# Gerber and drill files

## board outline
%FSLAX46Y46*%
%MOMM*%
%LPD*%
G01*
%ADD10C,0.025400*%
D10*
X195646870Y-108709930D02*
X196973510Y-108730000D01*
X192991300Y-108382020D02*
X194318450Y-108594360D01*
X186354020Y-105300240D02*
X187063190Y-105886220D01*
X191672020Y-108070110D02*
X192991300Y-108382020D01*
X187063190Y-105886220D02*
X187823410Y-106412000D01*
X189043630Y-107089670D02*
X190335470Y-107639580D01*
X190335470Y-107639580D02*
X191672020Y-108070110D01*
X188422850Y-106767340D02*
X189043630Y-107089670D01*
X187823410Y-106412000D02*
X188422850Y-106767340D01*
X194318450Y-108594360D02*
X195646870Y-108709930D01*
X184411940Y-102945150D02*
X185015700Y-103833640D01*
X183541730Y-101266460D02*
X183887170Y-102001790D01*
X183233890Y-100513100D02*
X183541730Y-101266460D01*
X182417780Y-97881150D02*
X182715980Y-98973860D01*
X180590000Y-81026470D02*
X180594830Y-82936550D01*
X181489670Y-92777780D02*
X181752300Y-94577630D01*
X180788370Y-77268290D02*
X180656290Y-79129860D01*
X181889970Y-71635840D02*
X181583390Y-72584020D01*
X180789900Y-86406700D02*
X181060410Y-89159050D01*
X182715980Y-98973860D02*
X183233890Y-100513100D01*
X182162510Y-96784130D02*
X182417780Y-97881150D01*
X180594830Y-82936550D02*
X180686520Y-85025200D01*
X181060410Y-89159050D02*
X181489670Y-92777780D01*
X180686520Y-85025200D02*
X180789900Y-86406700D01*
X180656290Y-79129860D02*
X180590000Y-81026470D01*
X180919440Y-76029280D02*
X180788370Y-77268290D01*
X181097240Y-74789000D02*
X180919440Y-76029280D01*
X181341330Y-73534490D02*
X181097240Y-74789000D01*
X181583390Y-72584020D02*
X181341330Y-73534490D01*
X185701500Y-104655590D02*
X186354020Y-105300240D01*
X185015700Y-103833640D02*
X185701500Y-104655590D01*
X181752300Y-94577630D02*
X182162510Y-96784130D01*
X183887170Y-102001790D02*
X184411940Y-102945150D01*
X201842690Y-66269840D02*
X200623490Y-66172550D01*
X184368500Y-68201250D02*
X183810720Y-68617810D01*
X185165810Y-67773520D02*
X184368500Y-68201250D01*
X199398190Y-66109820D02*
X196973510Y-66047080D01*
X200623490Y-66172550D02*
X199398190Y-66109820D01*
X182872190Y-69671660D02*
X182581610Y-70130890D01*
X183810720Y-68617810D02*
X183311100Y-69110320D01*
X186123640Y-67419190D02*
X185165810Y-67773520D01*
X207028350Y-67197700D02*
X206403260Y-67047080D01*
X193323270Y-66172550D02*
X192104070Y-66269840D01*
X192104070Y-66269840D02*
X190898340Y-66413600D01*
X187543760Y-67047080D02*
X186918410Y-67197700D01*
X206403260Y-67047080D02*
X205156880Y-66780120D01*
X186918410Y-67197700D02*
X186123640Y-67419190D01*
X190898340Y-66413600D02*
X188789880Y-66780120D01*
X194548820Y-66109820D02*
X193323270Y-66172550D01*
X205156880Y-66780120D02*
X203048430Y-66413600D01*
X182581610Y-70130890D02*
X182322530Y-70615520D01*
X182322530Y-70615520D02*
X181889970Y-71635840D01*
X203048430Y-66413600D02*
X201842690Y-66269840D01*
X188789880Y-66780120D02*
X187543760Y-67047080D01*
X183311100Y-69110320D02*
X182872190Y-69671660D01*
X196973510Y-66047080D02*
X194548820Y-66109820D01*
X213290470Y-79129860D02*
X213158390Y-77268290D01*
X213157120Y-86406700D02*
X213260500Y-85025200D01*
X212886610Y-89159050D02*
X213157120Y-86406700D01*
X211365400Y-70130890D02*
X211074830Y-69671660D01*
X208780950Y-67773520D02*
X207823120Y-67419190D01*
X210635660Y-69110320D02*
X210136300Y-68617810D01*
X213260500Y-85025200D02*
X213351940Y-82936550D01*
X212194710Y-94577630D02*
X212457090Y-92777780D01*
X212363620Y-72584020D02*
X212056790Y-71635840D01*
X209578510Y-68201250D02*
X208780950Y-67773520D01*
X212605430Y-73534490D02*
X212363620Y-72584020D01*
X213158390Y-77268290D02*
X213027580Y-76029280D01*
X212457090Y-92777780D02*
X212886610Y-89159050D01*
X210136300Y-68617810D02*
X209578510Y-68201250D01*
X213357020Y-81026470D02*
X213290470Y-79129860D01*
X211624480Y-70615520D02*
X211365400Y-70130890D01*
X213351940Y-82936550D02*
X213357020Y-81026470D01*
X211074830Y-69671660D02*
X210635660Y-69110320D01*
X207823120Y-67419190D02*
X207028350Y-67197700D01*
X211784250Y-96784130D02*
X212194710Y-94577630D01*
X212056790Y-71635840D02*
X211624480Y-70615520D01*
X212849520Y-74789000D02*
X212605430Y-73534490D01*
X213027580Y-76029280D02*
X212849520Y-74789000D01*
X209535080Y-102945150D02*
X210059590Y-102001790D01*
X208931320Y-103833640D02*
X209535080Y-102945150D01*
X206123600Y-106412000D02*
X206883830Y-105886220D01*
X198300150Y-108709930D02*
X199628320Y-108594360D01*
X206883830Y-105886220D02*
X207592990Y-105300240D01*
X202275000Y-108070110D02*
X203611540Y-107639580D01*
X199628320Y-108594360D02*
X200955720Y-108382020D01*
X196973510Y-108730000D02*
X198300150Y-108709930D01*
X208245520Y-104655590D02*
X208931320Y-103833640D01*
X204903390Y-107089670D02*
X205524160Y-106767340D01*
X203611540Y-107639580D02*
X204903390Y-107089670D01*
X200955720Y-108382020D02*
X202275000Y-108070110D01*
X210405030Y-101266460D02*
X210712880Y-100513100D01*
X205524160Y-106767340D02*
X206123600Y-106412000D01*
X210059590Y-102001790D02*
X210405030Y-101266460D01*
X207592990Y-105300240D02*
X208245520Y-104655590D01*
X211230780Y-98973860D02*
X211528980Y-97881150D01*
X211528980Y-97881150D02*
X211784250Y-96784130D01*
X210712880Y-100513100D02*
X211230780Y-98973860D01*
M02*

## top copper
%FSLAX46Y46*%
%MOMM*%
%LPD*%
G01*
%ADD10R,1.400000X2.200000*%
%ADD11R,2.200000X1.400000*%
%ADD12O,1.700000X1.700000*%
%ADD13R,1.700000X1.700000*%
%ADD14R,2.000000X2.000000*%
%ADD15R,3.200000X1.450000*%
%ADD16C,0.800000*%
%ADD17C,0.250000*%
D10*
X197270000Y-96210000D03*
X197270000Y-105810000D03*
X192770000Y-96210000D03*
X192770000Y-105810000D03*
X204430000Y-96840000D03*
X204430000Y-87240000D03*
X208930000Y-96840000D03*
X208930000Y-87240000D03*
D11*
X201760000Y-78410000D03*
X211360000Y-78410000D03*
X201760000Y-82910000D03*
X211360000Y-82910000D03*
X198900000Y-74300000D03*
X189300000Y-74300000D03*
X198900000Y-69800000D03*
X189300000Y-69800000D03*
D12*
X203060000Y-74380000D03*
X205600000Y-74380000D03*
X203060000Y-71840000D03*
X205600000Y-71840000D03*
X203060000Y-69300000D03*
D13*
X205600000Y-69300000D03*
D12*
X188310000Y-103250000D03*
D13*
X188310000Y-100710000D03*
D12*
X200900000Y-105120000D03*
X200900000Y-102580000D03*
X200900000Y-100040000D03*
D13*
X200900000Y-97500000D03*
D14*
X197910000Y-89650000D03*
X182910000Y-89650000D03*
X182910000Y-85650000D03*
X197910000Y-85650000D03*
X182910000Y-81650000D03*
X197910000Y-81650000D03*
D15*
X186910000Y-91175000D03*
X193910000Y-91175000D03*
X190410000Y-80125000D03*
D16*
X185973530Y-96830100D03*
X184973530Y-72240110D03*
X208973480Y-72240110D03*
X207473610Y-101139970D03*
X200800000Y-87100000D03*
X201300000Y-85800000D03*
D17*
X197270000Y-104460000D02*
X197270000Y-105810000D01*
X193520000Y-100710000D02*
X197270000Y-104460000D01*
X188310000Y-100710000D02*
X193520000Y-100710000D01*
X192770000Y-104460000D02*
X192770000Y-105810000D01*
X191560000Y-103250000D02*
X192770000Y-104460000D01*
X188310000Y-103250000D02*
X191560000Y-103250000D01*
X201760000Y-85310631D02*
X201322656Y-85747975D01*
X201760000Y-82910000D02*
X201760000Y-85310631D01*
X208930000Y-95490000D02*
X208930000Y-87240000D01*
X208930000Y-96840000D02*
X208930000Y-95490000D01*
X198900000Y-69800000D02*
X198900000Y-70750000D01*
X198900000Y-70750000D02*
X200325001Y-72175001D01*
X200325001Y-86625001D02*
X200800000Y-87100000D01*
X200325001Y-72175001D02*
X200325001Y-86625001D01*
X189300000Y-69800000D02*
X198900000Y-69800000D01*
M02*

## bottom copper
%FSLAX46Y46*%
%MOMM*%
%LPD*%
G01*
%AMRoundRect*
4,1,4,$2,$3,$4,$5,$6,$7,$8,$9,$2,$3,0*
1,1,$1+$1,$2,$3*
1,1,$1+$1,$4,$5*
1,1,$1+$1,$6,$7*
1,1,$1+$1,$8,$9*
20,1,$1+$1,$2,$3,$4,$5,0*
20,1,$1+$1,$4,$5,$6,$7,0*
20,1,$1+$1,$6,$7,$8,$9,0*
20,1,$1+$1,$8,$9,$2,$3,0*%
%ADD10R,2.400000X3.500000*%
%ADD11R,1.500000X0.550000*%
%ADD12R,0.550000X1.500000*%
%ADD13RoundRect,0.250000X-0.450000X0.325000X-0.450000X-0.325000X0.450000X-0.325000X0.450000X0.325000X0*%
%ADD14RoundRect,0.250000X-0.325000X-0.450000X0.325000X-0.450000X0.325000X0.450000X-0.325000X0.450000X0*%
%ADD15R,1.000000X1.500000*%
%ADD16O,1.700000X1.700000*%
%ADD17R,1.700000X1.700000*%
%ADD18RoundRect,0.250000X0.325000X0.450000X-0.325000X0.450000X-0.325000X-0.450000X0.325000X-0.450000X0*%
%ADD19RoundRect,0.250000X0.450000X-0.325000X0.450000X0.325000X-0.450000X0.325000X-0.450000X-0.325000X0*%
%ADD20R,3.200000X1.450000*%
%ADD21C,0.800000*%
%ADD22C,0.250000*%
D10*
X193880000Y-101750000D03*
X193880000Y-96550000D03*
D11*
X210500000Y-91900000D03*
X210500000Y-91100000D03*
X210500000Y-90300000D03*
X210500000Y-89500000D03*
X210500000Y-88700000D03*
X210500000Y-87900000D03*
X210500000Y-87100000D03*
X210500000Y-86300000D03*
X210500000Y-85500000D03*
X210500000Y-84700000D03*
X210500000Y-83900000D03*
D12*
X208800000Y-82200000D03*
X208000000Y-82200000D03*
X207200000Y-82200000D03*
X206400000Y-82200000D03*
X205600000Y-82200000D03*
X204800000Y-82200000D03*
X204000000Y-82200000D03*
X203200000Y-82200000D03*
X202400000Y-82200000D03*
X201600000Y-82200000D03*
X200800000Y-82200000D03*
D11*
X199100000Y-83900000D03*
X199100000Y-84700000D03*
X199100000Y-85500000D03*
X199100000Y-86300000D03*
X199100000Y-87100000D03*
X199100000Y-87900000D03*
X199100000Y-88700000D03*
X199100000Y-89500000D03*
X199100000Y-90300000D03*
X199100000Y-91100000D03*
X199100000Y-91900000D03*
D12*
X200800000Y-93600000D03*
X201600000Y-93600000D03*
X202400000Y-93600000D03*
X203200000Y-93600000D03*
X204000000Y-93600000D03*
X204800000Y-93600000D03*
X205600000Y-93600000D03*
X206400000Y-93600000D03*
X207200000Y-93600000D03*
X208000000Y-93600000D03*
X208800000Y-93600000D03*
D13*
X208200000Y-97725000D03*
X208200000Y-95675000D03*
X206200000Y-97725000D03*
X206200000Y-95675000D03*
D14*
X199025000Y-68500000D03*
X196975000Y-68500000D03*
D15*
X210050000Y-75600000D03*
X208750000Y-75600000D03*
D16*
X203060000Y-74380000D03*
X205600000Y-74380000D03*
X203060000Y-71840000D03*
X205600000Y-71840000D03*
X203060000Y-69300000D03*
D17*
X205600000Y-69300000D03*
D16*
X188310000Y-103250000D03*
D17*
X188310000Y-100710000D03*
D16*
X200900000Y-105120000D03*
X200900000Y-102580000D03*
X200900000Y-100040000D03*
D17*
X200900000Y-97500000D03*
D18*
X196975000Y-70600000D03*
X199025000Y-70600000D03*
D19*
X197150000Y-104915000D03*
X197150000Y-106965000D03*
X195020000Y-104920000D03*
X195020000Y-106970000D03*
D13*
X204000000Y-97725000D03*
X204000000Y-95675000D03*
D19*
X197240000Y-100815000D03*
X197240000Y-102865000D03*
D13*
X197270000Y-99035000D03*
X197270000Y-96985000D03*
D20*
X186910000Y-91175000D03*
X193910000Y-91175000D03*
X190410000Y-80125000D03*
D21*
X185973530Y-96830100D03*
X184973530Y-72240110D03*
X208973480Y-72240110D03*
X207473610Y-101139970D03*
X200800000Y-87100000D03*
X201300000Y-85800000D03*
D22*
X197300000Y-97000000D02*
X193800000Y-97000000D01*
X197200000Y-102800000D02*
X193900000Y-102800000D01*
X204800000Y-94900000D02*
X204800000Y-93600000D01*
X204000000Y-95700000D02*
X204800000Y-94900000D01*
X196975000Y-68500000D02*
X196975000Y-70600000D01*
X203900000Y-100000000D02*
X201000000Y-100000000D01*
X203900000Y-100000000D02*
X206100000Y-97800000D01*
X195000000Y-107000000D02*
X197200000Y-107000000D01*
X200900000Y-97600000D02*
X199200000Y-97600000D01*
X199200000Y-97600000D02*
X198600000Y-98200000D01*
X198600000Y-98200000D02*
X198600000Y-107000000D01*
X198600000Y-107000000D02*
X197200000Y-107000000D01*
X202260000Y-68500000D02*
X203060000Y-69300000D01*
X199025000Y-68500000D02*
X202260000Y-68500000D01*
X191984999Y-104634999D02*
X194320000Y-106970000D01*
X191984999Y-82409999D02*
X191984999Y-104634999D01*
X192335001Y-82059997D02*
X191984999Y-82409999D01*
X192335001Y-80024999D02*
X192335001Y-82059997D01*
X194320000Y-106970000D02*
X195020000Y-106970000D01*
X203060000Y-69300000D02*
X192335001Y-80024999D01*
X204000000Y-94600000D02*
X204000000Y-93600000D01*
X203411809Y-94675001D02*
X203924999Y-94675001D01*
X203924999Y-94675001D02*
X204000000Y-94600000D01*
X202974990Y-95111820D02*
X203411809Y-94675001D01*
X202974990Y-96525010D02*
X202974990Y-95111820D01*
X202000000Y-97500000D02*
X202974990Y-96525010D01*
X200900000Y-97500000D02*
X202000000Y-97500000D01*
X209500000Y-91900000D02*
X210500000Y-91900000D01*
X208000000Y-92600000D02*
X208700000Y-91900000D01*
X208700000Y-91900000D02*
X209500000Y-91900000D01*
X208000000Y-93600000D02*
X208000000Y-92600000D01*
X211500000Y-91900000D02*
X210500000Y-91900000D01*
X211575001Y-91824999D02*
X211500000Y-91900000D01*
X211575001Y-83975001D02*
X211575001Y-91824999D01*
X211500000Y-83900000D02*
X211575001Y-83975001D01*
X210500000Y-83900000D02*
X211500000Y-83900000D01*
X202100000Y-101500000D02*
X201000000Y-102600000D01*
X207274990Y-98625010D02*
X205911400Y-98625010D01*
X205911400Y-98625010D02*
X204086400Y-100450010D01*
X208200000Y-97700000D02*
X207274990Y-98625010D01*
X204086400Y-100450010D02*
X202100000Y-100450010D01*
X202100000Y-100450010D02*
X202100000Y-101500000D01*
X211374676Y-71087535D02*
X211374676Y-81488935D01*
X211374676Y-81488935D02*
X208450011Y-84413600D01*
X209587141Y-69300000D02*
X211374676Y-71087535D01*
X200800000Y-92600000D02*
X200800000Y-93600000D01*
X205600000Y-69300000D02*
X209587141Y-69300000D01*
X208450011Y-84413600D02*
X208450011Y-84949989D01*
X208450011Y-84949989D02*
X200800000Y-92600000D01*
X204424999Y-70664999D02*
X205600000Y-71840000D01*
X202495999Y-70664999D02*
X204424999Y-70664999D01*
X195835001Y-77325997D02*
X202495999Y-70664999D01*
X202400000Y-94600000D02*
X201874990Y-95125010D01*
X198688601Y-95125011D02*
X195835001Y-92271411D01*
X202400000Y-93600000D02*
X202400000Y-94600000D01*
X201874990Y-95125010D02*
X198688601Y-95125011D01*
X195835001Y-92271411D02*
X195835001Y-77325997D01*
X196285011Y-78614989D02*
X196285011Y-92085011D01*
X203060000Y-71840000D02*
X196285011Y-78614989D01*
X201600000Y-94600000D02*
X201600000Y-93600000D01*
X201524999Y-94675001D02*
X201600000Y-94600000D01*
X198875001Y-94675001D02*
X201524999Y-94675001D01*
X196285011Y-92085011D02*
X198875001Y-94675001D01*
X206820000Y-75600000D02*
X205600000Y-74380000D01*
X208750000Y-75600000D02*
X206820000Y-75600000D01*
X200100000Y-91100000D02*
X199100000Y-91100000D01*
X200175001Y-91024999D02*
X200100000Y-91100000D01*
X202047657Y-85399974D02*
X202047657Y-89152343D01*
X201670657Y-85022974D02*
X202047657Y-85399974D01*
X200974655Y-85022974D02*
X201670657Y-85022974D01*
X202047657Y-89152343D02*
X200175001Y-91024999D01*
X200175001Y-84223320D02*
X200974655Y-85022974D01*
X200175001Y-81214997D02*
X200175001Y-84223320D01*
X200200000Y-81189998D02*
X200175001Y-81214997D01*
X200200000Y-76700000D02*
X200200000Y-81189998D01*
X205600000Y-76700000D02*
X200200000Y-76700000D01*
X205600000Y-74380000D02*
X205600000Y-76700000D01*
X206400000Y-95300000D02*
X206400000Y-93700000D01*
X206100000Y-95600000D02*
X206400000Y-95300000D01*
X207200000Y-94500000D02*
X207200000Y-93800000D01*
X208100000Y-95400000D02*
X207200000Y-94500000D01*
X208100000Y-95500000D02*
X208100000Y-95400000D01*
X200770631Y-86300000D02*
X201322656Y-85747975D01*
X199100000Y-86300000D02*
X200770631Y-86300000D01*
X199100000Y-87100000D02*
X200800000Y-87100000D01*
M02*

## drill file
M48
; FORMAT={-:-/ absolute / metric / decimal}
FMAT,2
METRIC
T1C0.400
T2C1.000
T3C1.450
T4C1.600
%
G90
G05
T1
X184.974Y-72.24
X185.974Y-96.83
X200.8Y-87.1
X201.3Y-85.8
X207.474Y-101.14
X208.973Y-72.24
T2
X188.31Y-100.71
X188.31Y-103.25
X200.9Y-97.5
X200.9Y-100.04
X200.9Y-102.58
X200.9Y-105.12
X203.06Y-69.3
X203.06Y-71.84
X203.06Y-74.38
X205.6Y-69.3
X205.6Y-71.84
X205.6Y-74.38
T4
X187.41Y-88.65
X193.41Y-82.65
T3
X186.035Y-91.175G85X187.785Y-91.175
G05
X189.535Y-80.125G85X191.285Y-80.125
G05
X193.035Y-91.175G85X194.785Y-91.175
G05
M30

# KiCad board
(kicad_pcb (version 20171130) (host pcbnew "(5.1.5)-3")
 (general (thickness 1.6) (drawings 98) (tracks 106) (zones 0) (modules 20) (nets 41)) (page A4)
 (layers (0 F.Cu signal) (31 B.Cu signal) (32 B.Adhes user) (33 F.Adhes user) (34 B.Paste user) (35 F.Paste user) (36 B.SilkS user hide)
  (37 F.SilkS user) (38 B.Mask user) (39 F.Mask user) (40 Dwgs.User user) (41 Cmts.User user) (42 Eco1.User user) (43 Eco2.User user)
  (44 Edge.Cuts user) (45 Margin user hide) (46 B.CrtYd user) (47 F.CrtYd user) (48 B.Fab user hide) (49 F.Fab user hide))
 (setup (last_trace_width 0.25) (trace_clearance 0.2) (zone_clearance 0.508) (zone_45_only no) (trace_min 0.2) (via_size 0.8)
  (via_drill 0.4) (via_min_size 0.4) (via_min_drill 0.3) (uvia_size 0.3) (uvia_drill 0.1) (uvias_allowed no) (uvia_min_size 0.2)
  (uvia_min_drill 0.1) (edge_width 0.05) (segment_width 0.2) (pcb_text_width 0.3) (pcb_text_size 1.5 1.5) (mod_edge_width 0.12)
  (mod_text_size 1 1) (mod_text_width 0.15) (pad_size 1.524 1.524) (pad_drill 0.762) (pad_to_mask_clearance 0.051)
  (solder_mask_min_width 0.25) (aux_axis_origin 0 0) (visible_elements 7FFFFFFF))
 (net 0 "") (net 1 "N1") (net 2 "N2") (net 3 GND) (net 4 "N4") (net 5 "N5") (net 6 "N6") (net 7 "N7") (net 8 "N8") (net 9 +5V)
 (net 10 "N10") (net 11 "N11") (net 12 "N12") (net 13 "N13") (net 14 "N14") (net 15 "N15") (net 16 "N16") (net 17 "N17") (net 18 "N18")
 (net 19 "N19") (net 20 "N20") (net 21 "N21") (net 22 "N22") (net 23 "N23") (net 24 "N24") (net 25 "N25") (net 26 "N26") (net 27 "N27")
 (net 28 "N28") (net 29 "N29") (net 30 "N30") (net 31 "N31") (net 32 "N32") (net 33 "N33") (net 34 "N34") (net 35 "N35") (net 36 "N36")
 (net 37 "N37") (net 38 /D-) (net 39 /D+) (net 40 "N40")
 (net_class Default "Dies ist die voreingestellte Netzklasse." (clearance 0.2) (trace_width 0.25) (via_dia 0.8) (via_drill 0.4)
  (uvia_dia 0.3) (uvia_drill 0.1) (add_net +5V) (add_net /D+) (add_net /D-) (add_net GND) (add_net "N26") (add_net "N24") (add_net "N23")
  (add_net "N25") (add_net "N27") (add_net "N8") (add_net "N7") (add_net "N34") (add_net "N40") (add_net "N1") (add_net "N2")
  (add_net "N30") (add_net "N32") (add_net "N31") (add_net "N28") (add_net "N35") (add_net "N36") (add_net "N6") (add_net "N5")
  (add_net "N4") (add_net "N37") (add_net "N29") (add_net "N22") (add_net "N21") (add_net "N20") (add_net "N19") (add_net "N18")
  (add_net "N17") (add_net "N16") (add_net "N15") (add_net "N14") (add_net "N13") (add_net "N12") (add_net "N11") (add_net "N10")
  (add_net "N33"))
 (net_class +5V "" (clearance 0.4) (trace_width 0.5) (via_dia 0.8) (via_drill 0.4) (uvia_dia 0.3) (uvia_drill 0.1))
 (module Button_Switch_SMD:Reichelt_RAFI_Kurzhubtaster (layer F.Cu) (at 197.97 106.91 90)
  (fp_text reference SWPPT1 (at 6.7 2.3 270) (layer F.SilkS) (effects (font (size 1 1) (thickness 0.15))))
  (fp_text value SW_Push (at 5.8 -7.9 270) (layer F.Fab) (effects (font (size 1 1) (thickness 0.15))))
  (pad 2 smd rect (at 10.7 -0.7 90) (size 2.2 1.4) (layers F.Cu F.Paste F.Mask) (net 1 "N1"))
  (pad 2 smd rect (at 1.1 -0.7 90) (size 2.2 1.4) (layers F.Cu F.Paste F.Mask) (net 1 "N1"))
  (pad 1 smd rect (at 10.7 -5.2 90) (size 2.2 1.4) (layers F.Cu F.Paste F.Mask) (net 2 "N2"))
  (pad 1 smd rect (at 1.1 -5.2 90) (size 2.2 1.4) (layers F.Cu F.Paste F.Mask) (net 2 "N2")))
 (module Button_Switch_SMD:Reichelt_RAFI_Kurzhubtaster (layer F.Cu) (at 203.73 86.14 270)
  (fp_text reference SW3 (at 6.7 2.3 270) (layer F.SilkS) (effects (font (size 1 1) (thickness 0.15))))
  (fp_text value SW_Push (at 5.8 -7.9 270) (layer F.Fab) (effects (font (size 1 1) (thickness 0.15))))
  (pad 2 smd rect (at 10.7 -0.7 270) (size 2.2 1.4) (layers F.Cu F.Paste F.Mask) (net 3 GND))
  (pad 2 smd rect (at 1.1 -0.7 270) (size 2.2 1.4) (layers F.Cu F.Paste F.Mask) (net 3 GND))
  (pad 1 smd rect (at 10.7 -5.2 270) (size 2.2 1.4) (layers F.Cu F.Paste F.Mask) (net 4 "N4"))
  (pad 1 smd rect (at 1.1 -5.2 270) (size 2.2 1.4) (layers F.Cu F.Paste F.Mask) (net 4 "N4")))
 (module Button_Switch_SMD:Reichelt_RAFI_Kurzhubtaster (layer F.Cu) (at 212.46 77.71 180)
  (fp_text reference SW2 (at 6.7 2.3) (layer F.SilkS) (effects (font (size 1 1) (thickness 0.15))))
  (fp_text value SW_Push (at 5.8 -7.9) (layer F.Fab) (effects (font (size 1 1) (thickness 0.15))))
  (pad 2 smd rect (at 10.7 -0.7 180) (size 2.2 1.4) (layers F.Cu F.Paste F.Mask) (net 3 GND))
  (pad 2 smd rect (at 1.1 -0.7 180) (size 2.2 1.4) (layers F.Cu F.Paste F.Mask) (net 3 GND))
  (pad 1 smd rect (at 10.7 -5.2 180) (size 2.2 1.4) (layers F.Cu F.Paste F.Mask) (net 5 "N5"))
  (pad 1 smd rect (at 1.1 -5.2 180) (size 2.2 1.4) (layers F.Cu F.Paste F.Mask) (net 5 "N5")))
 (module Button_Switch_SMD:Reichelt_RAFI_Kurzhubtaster (layer F.Cu) (at 188.2 75)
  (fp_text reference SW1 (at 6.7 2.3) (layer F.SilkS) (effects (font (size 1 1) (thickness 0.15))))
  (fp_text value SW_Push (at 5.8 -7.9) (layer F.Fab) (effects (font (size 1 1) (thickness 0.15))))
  (pad 2 smd rect (at 10.7 -0.7) (size 2.2 1.4) (layers F.Cu F.Paste F.Mask) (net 3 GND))
  (pad 2 smd rect (at 1.1 -0.7) (size 2.2 1.4) (layers F.Cu F.Paste F.Mask) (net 3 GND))
  (pad 1 smd rect (at 10.7 -5.2) (size 2.2 1.4) (layers F.Cu F.Paste F.Mask) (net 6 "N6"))
  (pad 1 smd rect (at 1.1 -5.2) (size 2.2 1.4) (layers F.Cu F.Paste F.Mask) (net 6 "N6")))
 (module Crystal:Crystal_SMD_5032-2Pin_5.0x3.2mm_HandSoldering (layer B.Cu) (at 193.88 99.15 270)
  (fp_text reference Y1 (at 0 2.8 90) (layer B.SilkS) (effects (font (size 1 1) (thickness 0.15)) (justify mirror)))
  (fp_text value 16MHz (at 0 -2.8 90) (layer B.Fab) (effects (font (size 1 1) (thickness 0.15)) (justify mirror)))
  (pad 2 smd rect (at 2.6 0 270) (size 3.5 2.4) (layers B.Cu B.Paste B.Mask) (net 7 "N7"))
  (pad 1 smd rect (at -2.6 0 270) (size 3.5 2.4) (layers B.Cu B.Paste B.Mask) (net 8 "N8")))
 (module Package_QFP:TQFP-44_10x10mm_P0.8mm (layer B.Cu) (at 204.8 87.9 90)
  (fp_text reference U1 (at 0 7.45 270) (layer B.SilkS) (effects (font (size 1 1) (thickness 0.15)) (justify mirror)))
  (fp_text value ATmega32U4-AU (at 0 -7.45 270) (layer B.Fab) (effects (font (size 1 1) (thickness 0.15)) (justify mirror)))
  (pad 44 smd rect (at -4 5.7) (size 1.5 0.55) (layers B.Cu B.Paste B.Mask) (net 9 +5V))
  (pad 43 smd rect (at -3.2 5.7) (size 1.5 0.55) (layers B.Cu B.Paste B.Mask) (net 3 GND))
  (pad 42 smd rect (at -2.4 5.7) (size 1.5 0.55) (layers B.Cu B.Paste B.Mask) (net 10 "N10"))
  (pad 41 smd rect (at -1.6 5.7) (size 1.5 0.55) (layers B.Cu B.Paste B.Mask) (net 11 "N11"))
  (pad 40 smd rect (at -0.8 5.7) (size 1.5 0.55) (layers B.Cu B.Paste B.Mask) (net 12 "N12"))
  (pad 39 smd rect (at 0 5.7) (size 1.5 0.55) (layers B.Cu B.Paste B.Mask) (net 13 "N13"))
  (pad 38 smd rect (at 0.8 5.7) (size 1.5 0.55) (layers B.Cu B.Paste B.Mask) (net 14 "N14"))
  (pad 37 smd rect (at 1.6 5.7) (size 1.5 0.55) (layers B.Cu B.Paste B.Mask) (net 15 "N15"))
  (pad 36 smd rect (at 2.4 5.7) (size 1.5 0.55) (layers B.Cu B.Paste B.Mask) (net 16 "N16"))
  (pad 35 smd rect (at 3.2 5.7) (size 1.5 0.55) (layers B.Cu B.Paste B.Mask) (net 3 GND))
  (pad 34 smd rect (at 4 5.7) (size 1.5 0.55) (layers B.Cu B.Paste B.Mask) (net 9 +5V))
  (pad 33 smd rect (at 5.7 4 90) (size 1.5 0.55) (layers B.Cu B.Paste B.Mask) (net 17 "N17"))
  (pad 32 smd rect (at 5.7 3.2 90) (size 1.5 0.55) (layers B.Cu B.Paste B.Mask) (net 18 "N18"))
  (pad 31 smd rect (at 5.7 2.4 90) (size 1.5 0.55) (layers B.Cu B.Paste B.Mask) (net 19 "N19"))
  (pad 30 smd rect (at 5.7 1.6 90) (size 1.5 0.55) (layers B.Cu B.Paste B.Mask) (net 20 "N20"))
  (pad 29 smd rect (at 5.7 0.8 90) (size 1.5 0.55) (layers B.Cu B.Paste B.Mask) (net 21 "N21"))
  (pad 28 smd rect (at 5.7 0 90) (size 1.5 0.55) (layers B.Cu B.Paste B.Mask) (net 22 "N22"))
  (pad 27 smd rect (at 5.7 -0.8 90) (size 1.5 0.55) (layers B.Cu B.Paste B.Mask) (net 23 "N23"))
  (pad 26 smd rect (at 5.7 -1.6 90) (size 1.5 0.55) (layers B.Cu B.Paste B.Mask) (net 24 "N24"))
  (pad 25 smd rect (at 5.7 -2.4 90) (size 1.5 0.55) (layers B.Cu B.Paste B.Mask) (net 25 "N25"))
  (pad 24 smd rect (at 5.7 -3.2 90) (size 1.5 0.55) (layers B.Cu B.Paste B.Mask) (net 9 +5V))
  (pad 23 smd rect (at 5.7 -4 90) (size 1.5 0.55) (layers B.Cu B.Paste B.Mask) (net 3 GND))
  (pad 22 smd rect (at 4 -5.7) (size 1.5 0.55) (layers B.Cu B.Paste B.Mask) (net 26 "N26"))
  (pad 21 smd rect (at 3.2 -5.7) (size 1.5 0.55) (layers B.Cu B.Paste B.Mask) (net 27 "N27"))
  (pad 20 smd rect (at 2.4 -5.7) (size 1.5 0.55) (layers B.Cu B.Paste B.Mask) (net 4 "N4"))
  (pad 19 smd rect (at 1.6 -5.7) (size 1.5 0.55) (layers B.Cu B.Paste B.Mask) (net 5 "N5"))
  (pad 18 smd rect (at 0.8 -5.7) (size 1.5 0.55) (layers B.Cu B.Paste B.Mask) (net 6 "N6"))
  (pad 17 smd rect (at 0 -5.7) (size 1.5 0.55) (layers B.Cu B.Paste B.Mask) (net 8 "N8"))
  (pad 16 smd rect (at -0.8 -5.7) (size 1.5 0.55) (layers B.Cu B.Paste B.Mask) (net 7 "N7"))
  (pad 15 smd rect (at -1.6 -5.7) (size 1.5 0.55) (layers B.Cu B.Paste B.Mask) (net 3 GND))
  (pad 14 smd rect (at -2.4 -5.7) (size 1.5 0.55) (layers B.Cu B.Paste B.Mask) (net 9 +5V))
  (pad 13 smd rect (at -3.2 -5.7) (size 1.5 0.55) (layers B.Cu B.Paste B.Mask) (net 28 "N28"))
  (pad 12 smd rect (at -4 -5.7) (size 1.5 0.55) (layers B.Cu B.Paste B.Mask) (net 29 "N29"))
  (pad 11 smd rect (at -5.7 -4 90) (size 1.5 0.55) (layers B.Cu B.Paste B.Mask) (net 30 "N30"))
  (pad 10 smd rect (at -5.7 -3.2 90) (size 1.5 0.55) (layers B.Cu B.Paste B.Mask) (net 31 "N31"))
  (pad 9 smd rect (at -5.7 -2.4 90) (size 1.5 0.55) (layers B.Cu B.Paste B.Mask) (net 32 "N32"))
  (pad 8 smd rect (at -5.7 -1.6 90) (size 1.5 0.55) (layers B.Cu B.Paste B.Mask) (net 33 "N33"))
  (pad 7 smd rect (at -5.7 -0.8 90) (size 1.5 0.55) (layers B.Cu B.Paste B.Mask) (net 9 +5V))
  (pad 6 smd rect (at -5.7 0 90) (size 1.5 0.55) (layers B.Cu B.Paste B.Mask) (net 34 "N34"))
  (pad 5 smd rect (at -5.7 0.8 90) (size 1.5 0.55) (layers B.Cu B.Paste B.Mask) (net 3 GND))
  (pad 4 smd rect (at -5.7 1.6 90) (size 1.5 0.55) (layers B.Cu B.Paste B.Mask) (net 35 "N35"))
  (pad 3 smd rect (at -5.7 2.4 90) (size 1.5 0.55) (layers B.Cu B.Paste B.Mask) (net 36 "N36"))
  (pad 2 smd rect (at -5.7 3.2 90) (size 1.5 0.55) (layers B.Cu B.Paste B.Mask) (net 9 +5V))
  (pad 1 smd rect (at -5.7 4 90) (size 1.5 0.55) (layers B.Cu B.Paste B.Mask) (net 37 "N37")))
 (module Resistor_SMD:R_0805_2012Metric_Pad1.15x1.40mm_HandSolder (layer B.Cu) (at 208.2 96.7 270)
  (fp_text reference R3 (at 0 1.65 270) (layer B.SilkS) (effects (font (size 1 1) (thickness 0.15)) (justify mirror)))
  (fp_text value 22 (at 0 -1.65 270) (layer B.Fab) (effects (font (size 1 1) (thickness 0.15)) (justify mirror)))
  (pad 2 smd roundrect (at 1.025 0 270) (size 1.15 1.4) (layers B.Cu B.Paste B.Mask) (roundrect_rratio 0.217391) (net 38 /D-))
  (pad 1 smd roundrect (at -1.025 0 270) (size 1.15 1.4) (layers B.Cu B.Paste B.Mask) (roundrect_rratio 0.217391) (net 36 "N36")))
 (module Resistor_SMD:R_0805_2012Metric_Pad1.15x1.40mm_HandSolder (layer B.Cu) (at 206.2 96.7 270)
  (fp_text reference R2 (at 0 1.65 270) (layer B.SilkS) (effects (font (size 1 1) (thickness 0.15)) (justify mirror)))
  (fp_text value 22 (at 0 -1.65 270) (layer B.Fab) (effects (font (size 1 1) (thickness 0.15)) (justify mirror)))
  (pad 2 smd roundrect (at 1.025 0 270) (size 1.15 1.4) (layers B.Cu B.Paste B.Mask) (roundrect_rratio 0.217391) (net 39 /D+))
  (pad 1 smd roundrect (at -1.025 0 270) (size 1.15 1.4) (layers B.Cu B.Paste B.Mask) (roundrect_rratio 0.217391) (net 35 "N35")))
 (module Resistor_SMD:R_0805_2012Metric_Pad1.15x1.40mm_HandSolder (layer B.Cu) (at 198 68.5)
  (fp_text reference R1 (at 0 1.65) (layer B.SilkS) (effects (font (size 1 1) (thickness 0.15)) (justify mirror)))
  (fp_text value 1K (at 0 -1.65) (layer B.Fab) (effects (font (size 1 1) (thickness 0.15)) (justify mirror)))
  (pad 2 smd roundrect (at 1.025 0) (size 1.15 1.4) (layers B.Cu B.Paste B.Mask) (roundrect_rratio 0.217391) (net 9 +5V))
  (pad 1 smd roundrect (at -1.025 0) (size 1.15 1.4) (layers B.Cu B.Paste B.Mask) (roundrect_rratio 0.217391) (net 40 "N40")))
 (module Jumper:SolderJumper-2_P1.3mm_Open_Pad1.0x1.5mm (layer B.Cu) (at 209.4 75.6 180)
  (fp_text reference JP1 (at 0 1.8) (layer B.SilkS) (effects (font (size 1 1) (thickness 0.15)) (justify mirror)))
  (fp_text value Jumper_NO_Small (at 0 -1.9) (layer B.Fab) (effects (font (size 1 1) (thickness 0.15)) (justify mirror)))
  (pad 1 smd rect (at -0.65 0 180) (size 1 1.5) (layers B.Cu B.Mask) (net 3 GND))
  (pad 2 smd rect (at 0.65 0 180) (size 1 1.5) (layers B.Cu B.Mask) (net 28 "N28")))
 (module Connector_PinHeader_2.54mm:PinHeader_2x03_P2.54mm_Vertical (layer B.Cu) (at 205.6 69.3 180)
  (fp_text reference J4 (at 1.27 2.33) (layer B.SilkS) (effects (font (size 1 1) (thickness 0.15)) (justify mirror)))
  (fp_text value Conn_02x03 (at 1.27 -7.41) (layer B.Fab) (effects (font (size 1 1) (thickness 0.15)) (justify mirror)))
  (pad 6 thru_hole oval (at 2.54 -5.08 180) (size 1.7 1.7) (drill 1) (layers *.Cu *.Mask) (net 3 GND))
  (pad 5 thru_hole oval (at 0 -5.08 180) (size 1.7 1.7) (drill 1) (layers *.Cu *.Mask) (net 28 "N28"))
  (pad 4 thru_hole oval (at 2.54 -2.54 180) (size 1.7 1.7) (drill 1) (layers *.Cu *.Mask) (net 31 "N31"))
  (pad 3 thru_hole oval (at 0 -2.54 180) (size 1.7 1.7) (drill 1) (layers *.Cu *.Mask) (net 32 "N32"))
  (pad 2 thru_hole oval (at 2.54 0 180) (size 1.7 1.7) (drill 1) (layers *.Cu *.Mask) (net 9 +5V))
  (pad 1 thru_hole rect (at 0 0 180) (size 1.7 1.7) (drill 1) (layers *.Cu *.Mask) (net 30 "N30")))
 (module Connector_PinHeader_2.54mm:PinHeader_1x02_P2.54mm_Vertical (layer B.Cu) (at 188.31 100.71 180)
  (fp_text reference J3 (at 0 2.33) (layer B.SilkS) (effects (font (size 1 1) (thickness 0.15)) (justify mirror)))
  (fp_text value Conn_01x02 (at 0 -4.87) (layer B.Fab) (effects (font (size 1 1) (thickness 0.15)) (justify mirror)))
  (pad 2 thru_hole oval (at 0 -2.54 180) (size 1.7 1.7) (drill 1) (layers *.Cu *.Mask) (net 2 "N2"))
  (pad 1 thru_hole rect (at 0 0 180) (size 1.7 1.7) (drill 1) (layers *.Cu *.Mask) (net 1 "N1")))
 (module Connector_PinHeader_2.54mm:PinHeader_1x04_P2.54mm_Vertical (layer B.Cu) (at 200.9 97.5 180)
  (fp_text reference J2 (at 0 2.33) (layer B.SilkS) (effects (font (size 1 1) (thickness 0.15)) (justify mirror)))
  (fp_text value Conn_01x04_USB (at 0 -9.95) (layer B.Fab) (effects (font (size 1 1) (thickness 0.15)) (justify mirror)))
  (pad 4 thru_hole oval (at 0 -7.62 180) (size 1.7 1.7) (drill 1) (layers *.Cu *.Mask) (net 3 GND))
  (pad 3 thru_hole oval (at 0 -5.08 180) (size 1.7 1.7) (drill 1) (layers *.Cu *.Mask) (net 38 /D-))
  (pad 2 thru_hole oval (at 0 -2.54 180) (size 1.7 1.7) (drill 1) (layers *.Cu *.Mask) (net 39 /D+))
  (pad 1 thru_hole rect (at 0 0 180) (size 1.7 1.7) (drill 1) (layers *.Cu *.Mask) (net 9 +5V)))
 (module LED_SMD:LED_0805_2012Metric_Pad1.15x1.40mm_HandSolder (layer B.Cu) (at 198 70.6 180)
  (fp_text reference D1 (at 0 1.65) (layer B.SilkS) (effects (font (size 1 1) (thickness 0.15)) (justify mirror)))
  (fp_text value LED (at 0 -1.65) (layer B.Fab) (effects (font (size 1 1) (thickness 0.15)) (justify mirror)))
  (pad 2 smd roundrect (at 1.025 0 180) (size 1.15 1.4) (layers B.Cu B.Paste B.Mask) (roundrect_rratio 0.217391) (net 40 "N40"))
  (pad 1 smd roundrect (at -1.025 0 180) (size 1.15 1.4) (layers B.Cu B.Paste B.Mask) (roundrect_rratio 0.217391) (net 3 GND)))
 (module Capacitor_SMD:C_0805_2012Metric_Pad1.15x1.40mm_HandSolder (layer B.Cu) (at 197.15 105.94 90)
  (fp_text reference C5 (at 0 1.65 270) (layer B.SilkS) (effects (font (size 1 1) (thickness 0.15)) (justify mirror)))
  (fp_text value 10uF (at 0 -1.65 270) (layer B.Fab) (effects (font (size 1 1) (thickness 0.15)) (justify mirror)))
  (pad 2 smd roundrect (at 1.025 0 90) (size 1.15 1.4) (layers B.Cu B.Paste B.Mask) (roundrect_rratio 0.217391) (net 3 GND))
  (pad 1 smd roundrect (at -1.025 0 90) (size 1.15 1.4) (layers B.Cu B.Paste B.Mask) (roundrect_rratio 0.217391) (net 9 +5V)))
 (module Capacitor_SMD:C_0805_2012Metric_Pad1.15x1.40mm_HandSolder (layer B.Cu) (at 195.02 105.945 90)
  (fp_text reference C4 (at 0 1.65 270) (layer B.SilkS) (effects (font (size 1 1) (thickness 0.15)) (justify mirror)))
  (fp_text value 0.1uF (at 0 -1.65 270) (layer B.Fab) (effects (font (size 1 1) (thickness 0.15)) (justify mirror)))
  (pad 2 smd roundrect (at 1.025 0 90) (size 1.15 1.4) (layers B.Cu B.Paste B.Mask) (roundrect_rratio 0.217391) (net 3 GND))
  (pad 1 smd roundrect (at -1.025 0 90) (size 1.15 1.4) (layers B.Cu B.Paste B.Mask) (roundrect_rratio 0.217391) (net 9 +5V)))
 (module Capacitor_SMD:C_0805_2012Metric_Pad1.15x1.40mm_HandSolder (layer B.Cu) (at 204 96.7 270)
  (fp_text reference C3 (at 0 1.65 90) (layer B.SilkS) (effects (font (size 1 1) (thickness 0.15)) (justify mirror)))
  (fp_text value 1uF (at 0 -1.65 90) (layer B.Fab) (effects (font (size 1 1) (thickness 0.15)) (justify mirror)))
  (pad 2 smd roundrect (at 1.025 0 270) (size 1.15 1.4) (layers B.Cu B.Paste B.Mask) (roundrect_rratio 0.217391) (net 3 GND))
  (pad 1 smd roundrect (at -1.025 0 270) (size 1.15 1.4) (layers B.Cu B.Paste B.Mask) (roundrect_rratio 0.217391) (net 34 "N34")))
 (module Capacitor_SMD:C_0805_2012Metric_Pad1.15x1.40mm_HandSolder (layer B.Cu) (at 197.24 101.84 90)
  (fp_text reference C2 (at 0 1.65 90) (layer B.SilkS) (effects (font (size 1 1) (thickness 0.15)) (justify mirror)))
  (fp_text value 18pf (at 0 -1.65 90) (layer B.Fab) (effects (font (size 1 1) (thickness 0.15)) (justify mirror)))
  (pad 2 smd roundrect (at 1.025 0 90) (size 1.15 1.4) (layers B.Cu B.Paste B.Mask) (roundrect_rratio 0.217391) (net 3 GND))
  (pad 1 smd roundrect (at -1.025 0 90) (size 1.15 1.4) (layers B.Cu B.Paste B.Mask) (roundrect_rratio 0.217391) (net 7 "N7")))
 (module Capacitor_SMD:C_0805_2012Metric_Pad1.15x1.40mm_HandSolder (layer B.Cu) (at 197.27 98.01 270)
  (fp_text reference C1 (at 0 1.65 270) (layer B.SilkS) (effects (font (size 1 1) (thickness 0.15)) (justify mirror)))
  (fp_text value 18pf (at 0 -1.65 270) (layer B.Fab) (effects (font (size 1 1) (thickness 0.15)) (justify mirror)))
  (pad 2 smd roundrect (at 1.025 0 270) (size 1.15 1.4) (layers B.Cu B.Paste B.Mask) (roundrect_rratio 0.217391) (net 3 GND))
  (pad 1 smd roundrect (at -1.025 0 270) (size 1.15 1.4) (layers B.Cu B.Paste B.Mask) (roundrect_rratio 0.217391) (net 8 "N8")))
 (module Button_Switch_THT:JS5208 (layer F.Cu) (at 190.41 85.65)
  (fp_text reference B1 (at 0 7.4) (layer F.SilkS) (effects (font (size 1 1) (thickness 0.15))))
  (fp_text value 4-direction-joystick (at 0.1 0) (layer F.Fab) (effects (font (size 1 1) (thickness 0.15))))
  (pad 6 smd rect (at 7.5 4) (size 2 2) (layers F.Cu F.Paste F.Mask) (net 3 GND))
  (pad 3 smd rect (at -7.5 4) (size 2 2) (layers F.Cu F.Paste F.Mask) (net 23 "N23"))
  (pad 2 smd rect (at -7.5 0) (size 2 2) (layers F.Cu F.Paste F.Mask) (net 24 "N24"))
  (pad 5 smd rect (at 7.5 0) (size 2 2) (layers F.Cu F.Paste F.Mask) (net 27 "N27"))
  (pad 1 smd rect (at -7.5 -4) (size 2 2) (layers F.Cu F.Paste F.Mask) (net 26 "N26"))
  (pad 4 smd rect (at 7.5 -4) (size 2 2) (layers F.Cu F.Paste F.Mask) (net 25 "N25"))
  (pad "" np_thru_hole rect (at -3.5 5.525) (size 3.2 1.45) (drill oval 3.2 1.45) (layers *.Cu *.Mask))
  (pad "" np_thru_hole rect (at 3.5 5.525) (size 3.2 1.45) (drill oval 3.2 1.45) (layers *.Cu *.Mask))
  (pad "" np_thru_hole rect (at 0 -5.525) (size 3.2 1.45) (drill oval 3.2 1.45) (layers *.Cu *.Mask))
  (pad "" np_thru_hole circle (at -3 3) (size 1.6 1.6) (drill 1.6) (layers *.Cu *.Mask))
  (pad "" np_thru_hole circle (at 3 -3) (size 1.6 1.6) (drill 1.6) (layers *.Cu *.Mask)))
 (gr_line (start 195.64687 108.70993) (end 196.97351 108.73) (layer Edge.Cuts) (width 0.0254))
 (gr_line (start 192.9913 108.38202) (end 194.31845 108.59436) (layer Edge.Cuts) (width 0.0254))
 (gr_line (start 186.35402 105.30024) (end 187.06319 105.88622) (layer Edge.Cuts) (width 0.0254))
 (gr_line (start 191.67202 108.07011) (end 192.9913 108.38202) (layer Edge.Cuts) (width 0.0254))
 (gr_line (start 187.06319 105.88622) (end 187.82341 106.412) (layer Edge.Cuts) (width 0.0254))
 (gr_line (start 189.04363 107.08967) (end 190.33547 107.63958) (layer Edge.Cuts) (width 0.0254))
 (gr_line (start 190.33547 107.63958) (end 191.67202 108.07011) (layer Edge.Cuts) (width 0.0254))
 (gr_line (start 188.42285 106.76734) (end 189.04363 107.08967) (layer Edge.Cuts) (width 0.0254))
 (gr_line (start 187.82341 106.412) (end 188.42285 106.76734) (layer Edge.Cuts) (width 0.0254))
 (gr_line (start 194.31845 108.59436) (end 195.64687 108.70993) (layer Edge.Cuts) (width 0.0254))
 (gr_line (start 184.41194 102.94515) (end 185.0157 103.83364) (layer Edge.Cuts) (width 0.0254))
 (gr_line (start 183.54173 101.26646) (end 183.88717 102.00179) (layer Edge.Cuts) (width 0.0254))
 (gr_line (start 183.23389 100.5131) (end 183.54173 101.26646) (layer Edge.Cuts) (width 0.0254))
 (gr_line (start 182.41778 97.88115) (end 182.71598 98.97386) (layer Edge.Cuts) (width 0.0254))
 (gr_line (start 180.59 81.02647) (end 180.59483 82.93655) (layer Edge.Cuts) (width 0.0254))
 (gr_line (start 181.48967 92.77778) (end 181.7523 94.57763) (layer Edge.Cuts) (width 0.0254))
 (gr_line (start 180.78837 77.26829) (end 180.65629 79.12986) (layer Edge.Cuts) (width 0.0254))
 (gr_line (start 181.88997 71.63584) (end 181.58339 72.58402) (layer Edge.Cuts) (width 0.0254))
 (gr_line (start 180.7899 86.4067) (end 181.06041 89.15905) (layer Edge.Cuts) (width 0.0254))
 (gr_line (start 182.71598 98.97386) (end 183.23389 100.5131) (layer Edge.Cuts) (width 0.0254))
 (gr_line (start 182.16251 96.78413) (end 182.41778 97.88115) (layer Edge.Cuts) (width 0.0254))
 (gr_line (start 180.59483 82.93655) (end 180.68652 85.0252) (layer Edge.Cuts) (width 0.0254))
 (gr_line (start 181.06041 89.15905) (end 181.48967 92.77778) (layer Edge.Cuts) (width 0.0254))
 (gr_line (start 180.68652 85.0252) (end 180.7899 86.4067) (layer Edge.Cuts) (width 0.0254))
 (gr_line (start 180.65629 79.12986) (end 180.59 81.02647) (layer Edge.Cuts) (width 0.0254))
 (gr_line (start 180.91944 76.02928) (end 180.78837 77.26829) (layer Edge.Cuts) (width 0.0254))
 (gr_line (start 181.09724 74.789) (end 180.91944 76.02928) (layer Edge.Cuts) (width 0.0254))
 (gr_line (start 181.34133 73.53449) (end 181.09724 74.789) (layer Edge.Cuts) (width 0.0254))
 (gr_line (start 181.58339 72.58402) (end 181.34133 73.53449) (layer Edge.Cuts) (width 0.0254))
 (gr_line (start 185.7015 104.65559) (end 186.35402 105.30024) (layer Edge.Cuts) (width 0.0254))
 (gr_line (start 185.0157 103.83364) (end 185.7015 104.65559) (layer Edge.Cuts) (width 0.0254))
 (gr_line (start 181.7523 94.57763) (end 182.16251 96.78413) (layer Edge.Cuts) (width 0.0254))
 (gr_line (start 183.88717 102.00179) (end 184.41194 102.94515) (layer Edge.Cuts) (width 0.0254))
 (gr_line (start 201.84269 66.26984) (end 200.62349 66.17255) (layer Edge.Cuts) (width 0.0254))
 (gr_line (start 184.3685 68.20125) (end 183.81072 68.61781) (layer Edge.Cuts) (width 0.0254))
 (gr_line (start 185.16581 67.77352) (end 184.3685 68.20125) (layer Edge.Cuts) (width 0.0254))
 (gr_line (start 199.39819 66.10982) (end 196.97351 66.04708) (layer Edge.Cuts) (width 0.0254))
 (gr_line (start 200.62349 66.17255) (end 199.39819 66.10982) (layer Edge.Cuts) (width 0.0254))
 (gr_line (start 182.87219 69.67166) (end 182.58161 70.13089) (layer Edge.Cuts) (width 0.0254))
 (gr_line (start 183.81072 68.61781) (end 183.3111 69.11032) (layer Edge.Cuts) (width 0.0254))
 (gr_line (start 186.12364 67.41919) (end 185.16581 67.77352) (layer Edge.Cuts) (width 0.0254))
 (gr_line (start 207.02835 67.1977) (end 206.40326 67.04708) (layer Edge.Cuts) (width 0.0254))
 (gr_line (start 193.32327 66.17255) (end 192.10407 66.26984) (layer Edge.Cuts) (width 0.0254))
 (gr_line (start 192.10407 66.26984) (end 190.89834 66.4136) (layer Edge.Cuts) (width 0.0254))
 (gr_line (start 187.54376 67.04708) (end 186.91841 67.1977) (layer Edge.Cuts) (width 0.0254))
 (gr_line (start 206.40326 67.04708) (end 205.15688 66.78012) (layer Edge.Cuts) (width 0.0254))
 (gr_line (start 186.91841 67.1977) (end 186.12364 67.41919) (layer Edge.Cuts) (width 0.0254))
 (gr_line (start 190.89834 66.4136) (end 188.78988 66.78012) (layer Edge.Cuts) (width 0.0254))
 (gr_line (start 194.54882 66.10982) (end 193.32327 66.17255) (layer Edge.Cuts) (width 0.0254))
 (gr_line (start 205.15688 66.78012) (end 203.04843 66.4136) (layer Edge.Cuts) (width 0.0254))
 (gr_line (start 182.58161 70.13089) (end 182.32253 70.61552) (layer Edge.Cuts) (width 0.0254))
 (gr_line (start 182.32253 70.61552) (end 181.88997 71.63584) (layer Edge.Cuts) (width 0.0254))
 (gr_line (start 203.04843 66.4136) (end 201.84269 66.26984) (layer Edge.Cuts) (width 0.0254))
 (gr_line (start 188.78988 66.78012) (end 187.54376 67.04708) (layer Edge.Cuts) (width 0.0254))
 (gr_line (start 183.3111 69.11032) (end 182.87219 69.67166) (layer Edge.Cuts) (width 0.0254))
 (gr_line (start 196.97351 66.04708) (end 194.54882 66.10982) (layer Edge.Cuts) (width 0.0254))
 (gr_line (start 213.29047 79.12986) (end 213.15839 77.26829) (layer Edge.Cuts) (width 0.0254))
 (gr_line (start 213.15712 86.4067) (end 213.2605 85.0252) (layer Edge.Cuts) (width 0.0254))
 (gr_line (start 212.88661 89.15905) (end 213.15712 86.4067) (layer Edge.Cuts) (width 0.0254))
 (gr_line (start 211.3654 70.13089) (end 211.07483 69.67166) (layer Edge.Cuts) (width 0.0254))
 (gr_line (start 208.78095 67.77352) (end 207.82312 67.41919) (layer Edge.Cuts) (width 0.0254))
 (gr_line (start 210.63566 69.11032) (end 210.1363 68.61781) (layer Edge.Cuts) (width 0.0254))
 (gr_line (start 213.2605 85.0252) (end 213.35194 82.93655) (layer Edge.Cuts) (width 0.0254))
 (gr_line (start 212.19471 94.57763) (end 212.45709 92.77778) (layer Edge.Cuts) (width 0.0254))
 (gr_line (start 212.36362 72.58402) (end 212.05679 71.63584) (layer Edge.Cuts) (width 0.0254))
 (gr_line (start 209.57851 68.20125) (end 208.78095 67.77352) (layer Edge.Cuts) (width 0.0254))
 (gr_line (start 212.60543 73.53449) (end 212.36362 72.58402) (layer Edge.Cuts) (width 0.0254))
 (gr_line (start 213.15839 77.26829) (end 213.02758 76.02928) (layer Edge.Cuts) (width 0.0254))
 (gr_line (start 212.45709 92.77778) (end 212.88661 89.15905) (layer Edge.Cuts) (width 0.0254))
 (gr_line (start 210.1363 68.61781) (end 209.57851 68.20125) (layer Edge.Cuts) (width 0.0254))
 (gr_line (start 213.35702 81.02647) (end 213.29047 79.12986) (layer Edge.Cuts) (width 0.0254))
 (gr_line (start 211.62448 70.61552) (end 211.3654 70.13089) (layer Edge.Cuts) (width 0.0254))
 (gr_line (start 213.35194 82.93655) (end 213.35702 81.02647) (layer Edge.Cuts) (width 0.0254))
 (gr_line (start 211.07483 69.67166) (end 210.63566 69.11032) (layer Edge.Cuts) (width 0.0254))
 (gr_line (start 207.82312 67.41919) (end 207.02835 67.1977) (layer Edge.Cuts) (width 0.0254))
 (gr_line (start 211.78425 96.78413) (end 212.19471 94.57763) (layer Edge.Cuts) (width 0.0254))
 (gr_line (start 212.05679 71.63584) (end 211.62448 70.61552) (layer Edge.Cuts) (width 0.0254))
 (gr_line (start 212.84952 74.789) (end 212.60543 73.53449) (layer Edge.Cuts) (width 0.0254))
 (gr_line (start 213.02758 76.02928) (end 212.84952 74.789) (layer Edge.Cuts) (width 0.0254))
 (gr_line (start 209.53508 102.94515) (end 210.05959 102.00179) (layer Edge.Cuts) (width 0.0254))
 (gr_line (start 208.93132 103.83364) (end 209.53508 102.94515) (layer Edge.Cuts) (width 0.0254))
 (gr_line (start 206.1236 106.412) (end 206.88383 105.88622) (layer Edge.Cuts) (width 0.0254))
 (gr_line (start 198.30015 108.70993) (end 199.62832 108.59436) (layer Edge.Cuts) (width 0.0254))
 (gr_line (start 206.88383 105.88622) (end 207.59299 105.30024) (layer Edge.Cuts) (width 0.0254))
 (gr_line (start 202.275 108.07011) (end 203.61154 107.63958) (layer Edge.Cuts) (width 0.0254))
 (gr_line (start 199.62832 108.59436) (end 200.95572 108.38202) (layer Edge.Cuts) (width 0.0254))
 (gr_line (start 196.97351 108.73) (end 198.30015 108.70993) (layer Edge.Cuts) (width 0.0254))
 (gr_line (start 208.24552 104.65559) (end 208.93132 103.83364) (layer Edge.Cuts) (width 0.0254))
 (gr_line (start 204.90339 107.08967) (end 205.52416 106.76734) (layer Edge.Cuts) (width 0.0254))
 (gr_line (start 203.61154 107.63958) (end 204.90339 107.08967) (layer Edge.Cuts) (width 0.0254))
 (gr_line (start 200.95572 108.38202) (end 202.275 108.07011) (layer Edge.Cuts) (width 0.0254))
 (gr_line (start 210.40503 101.26646) (end 210.71288 100.5131) (layer Edge.Cuts) (width 0.0254))
 (gr_line (start 205.52416 106.76734) (end 206.1236 106.412) (layer Edge.Cuts) (width 0.0254))
 (gr_line (start 210.05959 102.00179) (end 210.40503 101.26646) (layer Edge.Cuts) (width 0.0254))
 (gr_line (start 207.59299 105.30024) (end 208.24552 104.65559) (layer Edge.Cuts) (width 0.0254))
 (gr_line (start 211.23078 98.97386) (end 211.52898 97.88115) (layer Edge.Cuts) (width 0.0254))
 (gr_line (start 211.52898 97.88115) (end 211.78425 96.78413) (layer Edge.Cuts) (width 0.0254))
 (gr_line (start 210.71288 100.5131) (end 211.23078 98.97386) (layer Edge.Cuts) (width 0.0254))
 (via (at 185.97353 96.8301) (size 0.8) (drill 0.4) (layers F.Cu B.Cu) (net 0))
 (via (at 184.97353 72.24011) (size 0.8) (drill 0.4) (layers F.Cu B.Cu) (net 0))
 (via (at 208.97348 72.24011) (size 0.8) (drill 0.4) (layers F.Cu B.Cu) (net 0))
 (via (at 207.47361 101.13997) (size 0.8) (drill 0.4) (layers F.Cu B.Cu) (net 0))
 (via (at 200.8 87.1) (size 0.8) (drill 0.4) (layers F.Cu B.Cu) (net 6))
 (segment (start 197.3 97) (end 193.8 97) (width 0.25) (layer B.Cu) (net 8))
 (segment (start 197.2 102.8) (end 193.9 102.8) (width 0.25) (layer B.Cu) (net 7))
 (segment (start 204.8 94.9) (end 204.8 93.6) (width 0.25) (layer B.Cu) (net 34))
 (segment (start 204 95.7) (end 204.8 94.9) (width 0.25) (layer B.Cu) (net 34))
 (segment (start 196.975 68.5) (end 196.975 70.6) (width 0.25) (layer B.Cu) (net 40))
 (segment (start 203.9 100) (end 201 100) (width 0.25) (layer B.Cu) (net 39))
 (segment (start 203.9 100) (end 206.1 97.8) (width 0.25) (layer B.Cu) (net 39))
 (segment (start 195 107) (end 197.2 107) (width 0.25) (layer B.Cu) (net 9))
 (segment (start 200.9 97.6) (end 199.2 97.6) (width 0.25) (layer B.Cu) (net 9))
 (segment (start 199.2 97.6) (end 198.6 98.2) (width 0.25) (layer B.Cu) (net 9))
 (segment (start 198.6 98.2) (end 198.6 107) (width 0.25) (layer B.Cu) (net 9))
 (segment (start 198.6 107) (end 197.2 107) (width 0.25) (layer B.Cu) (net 9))
 (segment (start 202.26 68.5) (end 203.06 69.3) (width 0.25) (layer B.Cu) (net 9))
 (segment (start 199.025 68.5) (end 202.26 68.5) (width 0.25) (layer B.Cu) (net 9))
 (segment (start 191.984999 104.634999) (end 194.32 106.97) (width 0.25) (layer B.Cu) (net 9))
 (segment (start 191.984999 82.409999) (end 191.984999 104.634999) (width 0.25) (layer B.Cu) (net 9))
 (segment (start 192.335001 82.059997) (end 191.984999 82.409999) (width 0.25) (layer B.Cu) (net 9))
 (segment (start 192.335001 80.024999) (end 192.335001 82.059997) (width 0.25) (layer B.Cu) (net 9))
 (segment (start 194.32 106.97) (end 195.02 106.97) (width 0.25) (layer B.Cu) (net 9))
 (segment (start 203.06 69.3) (end 192.335001 80.024999) (width 0.25) (layer B.Cu) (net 9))
 (segment (start 204 94.6) (end 204 93.6) (width 0.25) (layer B.Cu) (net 9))
 (segment (start 203.411809 94.675001) (end 203.924999 94.675001) (width 0.25) (layer B.Cu) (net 9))
 (segment (start 203.924999 94.675001) (end 204 94.6) (width 0.25) (layer B.Cu) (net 9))
 (segment (start 202.97499 95.11182) (end 203.411809 94.675001) (width 0.25) (layer B.Cu) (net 9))
 (segment (start 202.97499 96.52501) (end 202.97499 95.11182) (width 0.25) (layer B.Cu) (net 9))
 (segment (start 202 97.5) (end 202.97499 96.52501) (width 0.25) (layer B.Cu) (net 9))
 (segment (start 200.9 97.5) (end 202 97.5) (width 0.25) (layer B.Cu) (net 9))
 (segment (start 209.5 91.9) (end 210.5 91.9) (width 0.25) (layer B.Cu) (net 9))
 (segment (start 208 92.6) (end 208.7 91.9) (width 0.25) (layer B.Cu) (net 9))
 (segment (start 208.7 91.9) (end 209.5 91.9) (width 0.25) (layer B.Cu) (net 9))
 (segment (start 208 93.6) (end 208 92.6) (width 0.25) (layer B.Cu) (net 9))
 (segment (start 211.5 91.9) (end 210.5 91.9) (width 0.25) (layer B.Cu) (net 9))
 (segment (start 211.575001 91.824999) (end 211.5 91.9) (width 0.25) (layer B.Cu) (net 9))
 (segment (start 211.575001 83.975001) (end 211.575001 91.824999) (width 0.25) (layer B.Cu) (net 9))
 (segment (start 211.5 83.9) (end 211.575001 83.975001) (width 0.25) (layer B.Cu) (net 9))
 (segment (start 210.5 83.9) (end 211.5 83.9) (width 0.25) (layer B.Cu) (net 9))
 (segment (start 202.1 101.5) (end 201 102.6) (width 0.25) (layer B.Cu) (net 38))
 (segment (start 207.27499 98.62501) (end 205.9114 98.62501) (width 0.25) (layer B.Cu) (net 38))
 (segment (start 205.9114 98.62501) (end 204.0864 100.45001) (width 0.25) (layer B.Cu) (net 38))
 (segment (start 208.2 97.7) (end 207.27499 98.62501) (width 0.25) (layer B.Cu) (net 38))
 (segment (start 204.0864 100.45001) (end 202.1 100.45001) (width 0.25) (layer B.Cu) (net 38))
 (segment (start 202.1 100.45001) (end 202.1 101.5) (width 0.25) (layer B.Cu) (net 38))
 (segment (start 197.27 104.46) (end 197.27 105.81) (width 0.25) (layer F.Cu) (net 1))
 (segment (start 193.52 100.71) (end 197.27 104.46) (width 0.25) (layer F.Cu) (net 1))
 (segment (start 188.31 100.71) (end 193.52 100.71) (width 0.25) (layer F.Cu) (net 1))
 (segment (start 192.77 104.46) (end 192.77 105.81) (width 0.25) (layer F.Cu) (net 2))
 (segment (start 191.56 103.25) (end 192.77 104.46) (width 0.25) (layer F.Cu) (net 2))
 (segment (start 188.31 103.25) (end 191.56 103.25) (width 0.25) (layer F.Cu) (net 2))
 (segment (start 211.374676 71.087535) (end 211.374676 81.488935) (width 0.25) (layer B.Cu) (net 30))
 (segment (start 211.374676 81.488935) (end 208.450011 84.4136) (width 0.25) (layer B.Cu) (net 30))
 (segment (start 209.587141 69.3) (end 211.374676 71.087535) (width 0.25) (layer B.Cu) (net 30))
 (segment (start 200.8 92.6) (end 200.8 93.6) (width 0.25) (layer B.Cu) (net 30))
 (segment (start 205.6 69.3) (end 209.587141 69.3) (width 0.25) (layer B.Cu) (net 30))
 (segment (start 208.450011 84.4136) (end 208.450011 84.949989) (width 0.25) (layer B.Cu) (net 30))
 (segment (start 208.450011 84.949989) (end 200.8 92.6) (width 0.25) (layer B.Cu) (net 30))
 (segment (start 204.424999 70.664999) (end 205.6 71.84) (width 0.25) (layer B.Cu) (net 32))
 (segment (start 202.495999 70.664999) (end 204.424999 70.664999) (width 0.25) (layer B.Cu) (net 32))
 (segment (start 195.835001 77.325997) (end 202.495999 70.664999) (width 0.25) (layer B.Cu) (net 32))
 (segment (start 202.4 94.6) (end 201.87499 95.12501) (width 0.25) (layer B.Cu) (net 32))
 (segment (start 198.688601 95.125011) (end 195.835001 92.271411) (width 0.25) (layer B.Cu) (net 32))
 (segment (start 202.4 93.6) (end 202.4 94.6) (width 0.25) (layer B.Cu) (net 32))
 (segment (start 201.87499 95.12501) (end 198.688601 95.125011) (width 0.25) (layer B.Cu) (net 32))
 (segment (start 195.835001 92.271411) (end 195.835001 77.325997) (width 0.25) (layer B.Cu) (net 32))
 (segment (start 196.285011 78.614989) (end 196.285011 92.085011) (width 0.25) (layer B.Cu) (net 31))
 (segment (start 203.06 71.84) (end 196.285011 78.614989) (width 0.25) (layer B.Cu) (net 31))
 (segment (start 201.6 94.6) (end 201.6 93.6) (width 0.25) (layer B.Cu) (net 31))
 (segment (start 201.524999 94.675001) (end 201.6 94.6) (width 0.25) (layer B.Cu) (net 31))
 (segment (start 198.875001 94.675001) (end 201.524999 94.675001) (width 0.25) (layer B.Cu) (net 31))
 (segment (start 196.285011 92.085011) (end 198.875001 94.675001) (width 0.25) (layer B.Cu) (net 31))
 (segment (start 206.82 75.6) (end 205.6 74.38) (width 0.25) (layer B.Cu) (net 28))
 (segment (start 208.75 75.6) (end 206.82 75.6) (width 0.25) (layer B.Cu) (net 28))
 (segment (start 200.1 91.1) (end 199.1 91.1) (width 0.25) (layer B.Cu) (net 28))
 (segment (start 200.175001 91.024999) (end 200.1 91.1) (width 0.25) (layer B.Cu) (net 28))
 (segment (start 202.047657 85.399974) (end 202.047657 89.152343) (width 0.25) (layer B.Cu) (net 28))
 (segment (start 201.670657 85.022974) (end 202.047657 85.399974) (width 0.25) (layer B.Cu) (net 28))
 (segment (start 200.974655 85.022974) (end 201.670657 85.022974) (width 0.25) (layer B.Cu) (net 28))
 (segment (start 202.047657 89.152343) (end 200.175001 91.024999) (width 0.25) (layer B.Cu) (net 28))
 (segment (start 200.175001 84.22332) (end 200.974655 85.022974) (width 0.25) (layer B.Cu) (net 28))
 (segment (start 200.175001 81.214997) (end 200.175001 84.22332) (width 0.25) (layer B.Cu) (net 28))
 (segment (start 200.2 81.189998) (end 200.175001 81.214997) (width 0.25) (layer B.Cu) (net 28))
 (segment (start 200.2 76.7) (end 200.2 81.189998) (width 0.25) (layer B.Cu) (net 28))
 (segment (start 205.6 76.7) (end 200.2 76.7) (width 0.25) (layer B.Cu) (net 28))
 (segment (start 205.6 74.38) (end 205.6 76.7) (width 0.25) (layer B.Cu) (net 28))
 (segment (start 206.4 95.3) (end 206.4 93.7) (width 0.25) (layer B.Cu) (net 35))
 (segment (start 206.1 95.6) (end 206.4 95.3) (width 0.25) (layer B.Cu) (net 35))
 (segment (start 207.2 94.5) (end 207.2 93.8) (width 0.25) (layer B.Cu) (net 36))
 (segment (start 208.1 95.4) (end 207.2 94.5) (width 0.25) (layer B.Cu) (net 36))
 (segment (start 208.1 95.5) (end 208.1 95.4) (width 0.25) (layer B.Cu) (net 36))
 (segment (start 201.76 85.310631) (end 201.322656 85.747975) (width 0.25) (layer F.Cu) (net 5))
 (segment (start 201.76 82.91) (end 201.76 85.310631) (width 0.25) (layer F.Cu) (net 5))
 (via (at 201.3 85.8) (size 0.8) (drill 0.4) (layers F.Cu B.Cu) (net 5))
 (segment (start 200.770631 86.3) (end 201.322656 85.747975) (width 0.25) (layer B.Cu) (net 5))
 (segment (start 199.1 86.3) (end 200.770631 86.3) (width 0.25) (layer B.Cu) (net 5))
 (segment (start 208.93 95.49) (end 208.93 87.24) (width 0.25) (layer F.Cu) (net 4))
 (segment (start 208.93 96.84) (end 208.93 95.49) (width 0.25) (layer F.Cu) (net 4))
 (segment (start 198.9 69.8) (end 198.9 70.75) (width 0.25) (layer F.Cu) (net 6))
 (segment (start 198.9 70.75) (end 200.325001 72.175001) (width 0.25) (layer F.Cu) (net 6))
 (segment (start 199.1 87.1) (end 200.8 87.1) (width 0.25) (layer B.Cu) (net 6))
 (segment (start 200.325001 86.625001) (end 200.8 87.1) (width 0.25) (layer F.Cu) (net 6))
 (segment (start 200.325001 72.175001) (end 200.325001 86.625001) (width 0.25) (layer F.Cu) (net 6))
 (segment (start 189.3 69.8) (end 198.9 69.8) (width 0.25) (layer F.Cu) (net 6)))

